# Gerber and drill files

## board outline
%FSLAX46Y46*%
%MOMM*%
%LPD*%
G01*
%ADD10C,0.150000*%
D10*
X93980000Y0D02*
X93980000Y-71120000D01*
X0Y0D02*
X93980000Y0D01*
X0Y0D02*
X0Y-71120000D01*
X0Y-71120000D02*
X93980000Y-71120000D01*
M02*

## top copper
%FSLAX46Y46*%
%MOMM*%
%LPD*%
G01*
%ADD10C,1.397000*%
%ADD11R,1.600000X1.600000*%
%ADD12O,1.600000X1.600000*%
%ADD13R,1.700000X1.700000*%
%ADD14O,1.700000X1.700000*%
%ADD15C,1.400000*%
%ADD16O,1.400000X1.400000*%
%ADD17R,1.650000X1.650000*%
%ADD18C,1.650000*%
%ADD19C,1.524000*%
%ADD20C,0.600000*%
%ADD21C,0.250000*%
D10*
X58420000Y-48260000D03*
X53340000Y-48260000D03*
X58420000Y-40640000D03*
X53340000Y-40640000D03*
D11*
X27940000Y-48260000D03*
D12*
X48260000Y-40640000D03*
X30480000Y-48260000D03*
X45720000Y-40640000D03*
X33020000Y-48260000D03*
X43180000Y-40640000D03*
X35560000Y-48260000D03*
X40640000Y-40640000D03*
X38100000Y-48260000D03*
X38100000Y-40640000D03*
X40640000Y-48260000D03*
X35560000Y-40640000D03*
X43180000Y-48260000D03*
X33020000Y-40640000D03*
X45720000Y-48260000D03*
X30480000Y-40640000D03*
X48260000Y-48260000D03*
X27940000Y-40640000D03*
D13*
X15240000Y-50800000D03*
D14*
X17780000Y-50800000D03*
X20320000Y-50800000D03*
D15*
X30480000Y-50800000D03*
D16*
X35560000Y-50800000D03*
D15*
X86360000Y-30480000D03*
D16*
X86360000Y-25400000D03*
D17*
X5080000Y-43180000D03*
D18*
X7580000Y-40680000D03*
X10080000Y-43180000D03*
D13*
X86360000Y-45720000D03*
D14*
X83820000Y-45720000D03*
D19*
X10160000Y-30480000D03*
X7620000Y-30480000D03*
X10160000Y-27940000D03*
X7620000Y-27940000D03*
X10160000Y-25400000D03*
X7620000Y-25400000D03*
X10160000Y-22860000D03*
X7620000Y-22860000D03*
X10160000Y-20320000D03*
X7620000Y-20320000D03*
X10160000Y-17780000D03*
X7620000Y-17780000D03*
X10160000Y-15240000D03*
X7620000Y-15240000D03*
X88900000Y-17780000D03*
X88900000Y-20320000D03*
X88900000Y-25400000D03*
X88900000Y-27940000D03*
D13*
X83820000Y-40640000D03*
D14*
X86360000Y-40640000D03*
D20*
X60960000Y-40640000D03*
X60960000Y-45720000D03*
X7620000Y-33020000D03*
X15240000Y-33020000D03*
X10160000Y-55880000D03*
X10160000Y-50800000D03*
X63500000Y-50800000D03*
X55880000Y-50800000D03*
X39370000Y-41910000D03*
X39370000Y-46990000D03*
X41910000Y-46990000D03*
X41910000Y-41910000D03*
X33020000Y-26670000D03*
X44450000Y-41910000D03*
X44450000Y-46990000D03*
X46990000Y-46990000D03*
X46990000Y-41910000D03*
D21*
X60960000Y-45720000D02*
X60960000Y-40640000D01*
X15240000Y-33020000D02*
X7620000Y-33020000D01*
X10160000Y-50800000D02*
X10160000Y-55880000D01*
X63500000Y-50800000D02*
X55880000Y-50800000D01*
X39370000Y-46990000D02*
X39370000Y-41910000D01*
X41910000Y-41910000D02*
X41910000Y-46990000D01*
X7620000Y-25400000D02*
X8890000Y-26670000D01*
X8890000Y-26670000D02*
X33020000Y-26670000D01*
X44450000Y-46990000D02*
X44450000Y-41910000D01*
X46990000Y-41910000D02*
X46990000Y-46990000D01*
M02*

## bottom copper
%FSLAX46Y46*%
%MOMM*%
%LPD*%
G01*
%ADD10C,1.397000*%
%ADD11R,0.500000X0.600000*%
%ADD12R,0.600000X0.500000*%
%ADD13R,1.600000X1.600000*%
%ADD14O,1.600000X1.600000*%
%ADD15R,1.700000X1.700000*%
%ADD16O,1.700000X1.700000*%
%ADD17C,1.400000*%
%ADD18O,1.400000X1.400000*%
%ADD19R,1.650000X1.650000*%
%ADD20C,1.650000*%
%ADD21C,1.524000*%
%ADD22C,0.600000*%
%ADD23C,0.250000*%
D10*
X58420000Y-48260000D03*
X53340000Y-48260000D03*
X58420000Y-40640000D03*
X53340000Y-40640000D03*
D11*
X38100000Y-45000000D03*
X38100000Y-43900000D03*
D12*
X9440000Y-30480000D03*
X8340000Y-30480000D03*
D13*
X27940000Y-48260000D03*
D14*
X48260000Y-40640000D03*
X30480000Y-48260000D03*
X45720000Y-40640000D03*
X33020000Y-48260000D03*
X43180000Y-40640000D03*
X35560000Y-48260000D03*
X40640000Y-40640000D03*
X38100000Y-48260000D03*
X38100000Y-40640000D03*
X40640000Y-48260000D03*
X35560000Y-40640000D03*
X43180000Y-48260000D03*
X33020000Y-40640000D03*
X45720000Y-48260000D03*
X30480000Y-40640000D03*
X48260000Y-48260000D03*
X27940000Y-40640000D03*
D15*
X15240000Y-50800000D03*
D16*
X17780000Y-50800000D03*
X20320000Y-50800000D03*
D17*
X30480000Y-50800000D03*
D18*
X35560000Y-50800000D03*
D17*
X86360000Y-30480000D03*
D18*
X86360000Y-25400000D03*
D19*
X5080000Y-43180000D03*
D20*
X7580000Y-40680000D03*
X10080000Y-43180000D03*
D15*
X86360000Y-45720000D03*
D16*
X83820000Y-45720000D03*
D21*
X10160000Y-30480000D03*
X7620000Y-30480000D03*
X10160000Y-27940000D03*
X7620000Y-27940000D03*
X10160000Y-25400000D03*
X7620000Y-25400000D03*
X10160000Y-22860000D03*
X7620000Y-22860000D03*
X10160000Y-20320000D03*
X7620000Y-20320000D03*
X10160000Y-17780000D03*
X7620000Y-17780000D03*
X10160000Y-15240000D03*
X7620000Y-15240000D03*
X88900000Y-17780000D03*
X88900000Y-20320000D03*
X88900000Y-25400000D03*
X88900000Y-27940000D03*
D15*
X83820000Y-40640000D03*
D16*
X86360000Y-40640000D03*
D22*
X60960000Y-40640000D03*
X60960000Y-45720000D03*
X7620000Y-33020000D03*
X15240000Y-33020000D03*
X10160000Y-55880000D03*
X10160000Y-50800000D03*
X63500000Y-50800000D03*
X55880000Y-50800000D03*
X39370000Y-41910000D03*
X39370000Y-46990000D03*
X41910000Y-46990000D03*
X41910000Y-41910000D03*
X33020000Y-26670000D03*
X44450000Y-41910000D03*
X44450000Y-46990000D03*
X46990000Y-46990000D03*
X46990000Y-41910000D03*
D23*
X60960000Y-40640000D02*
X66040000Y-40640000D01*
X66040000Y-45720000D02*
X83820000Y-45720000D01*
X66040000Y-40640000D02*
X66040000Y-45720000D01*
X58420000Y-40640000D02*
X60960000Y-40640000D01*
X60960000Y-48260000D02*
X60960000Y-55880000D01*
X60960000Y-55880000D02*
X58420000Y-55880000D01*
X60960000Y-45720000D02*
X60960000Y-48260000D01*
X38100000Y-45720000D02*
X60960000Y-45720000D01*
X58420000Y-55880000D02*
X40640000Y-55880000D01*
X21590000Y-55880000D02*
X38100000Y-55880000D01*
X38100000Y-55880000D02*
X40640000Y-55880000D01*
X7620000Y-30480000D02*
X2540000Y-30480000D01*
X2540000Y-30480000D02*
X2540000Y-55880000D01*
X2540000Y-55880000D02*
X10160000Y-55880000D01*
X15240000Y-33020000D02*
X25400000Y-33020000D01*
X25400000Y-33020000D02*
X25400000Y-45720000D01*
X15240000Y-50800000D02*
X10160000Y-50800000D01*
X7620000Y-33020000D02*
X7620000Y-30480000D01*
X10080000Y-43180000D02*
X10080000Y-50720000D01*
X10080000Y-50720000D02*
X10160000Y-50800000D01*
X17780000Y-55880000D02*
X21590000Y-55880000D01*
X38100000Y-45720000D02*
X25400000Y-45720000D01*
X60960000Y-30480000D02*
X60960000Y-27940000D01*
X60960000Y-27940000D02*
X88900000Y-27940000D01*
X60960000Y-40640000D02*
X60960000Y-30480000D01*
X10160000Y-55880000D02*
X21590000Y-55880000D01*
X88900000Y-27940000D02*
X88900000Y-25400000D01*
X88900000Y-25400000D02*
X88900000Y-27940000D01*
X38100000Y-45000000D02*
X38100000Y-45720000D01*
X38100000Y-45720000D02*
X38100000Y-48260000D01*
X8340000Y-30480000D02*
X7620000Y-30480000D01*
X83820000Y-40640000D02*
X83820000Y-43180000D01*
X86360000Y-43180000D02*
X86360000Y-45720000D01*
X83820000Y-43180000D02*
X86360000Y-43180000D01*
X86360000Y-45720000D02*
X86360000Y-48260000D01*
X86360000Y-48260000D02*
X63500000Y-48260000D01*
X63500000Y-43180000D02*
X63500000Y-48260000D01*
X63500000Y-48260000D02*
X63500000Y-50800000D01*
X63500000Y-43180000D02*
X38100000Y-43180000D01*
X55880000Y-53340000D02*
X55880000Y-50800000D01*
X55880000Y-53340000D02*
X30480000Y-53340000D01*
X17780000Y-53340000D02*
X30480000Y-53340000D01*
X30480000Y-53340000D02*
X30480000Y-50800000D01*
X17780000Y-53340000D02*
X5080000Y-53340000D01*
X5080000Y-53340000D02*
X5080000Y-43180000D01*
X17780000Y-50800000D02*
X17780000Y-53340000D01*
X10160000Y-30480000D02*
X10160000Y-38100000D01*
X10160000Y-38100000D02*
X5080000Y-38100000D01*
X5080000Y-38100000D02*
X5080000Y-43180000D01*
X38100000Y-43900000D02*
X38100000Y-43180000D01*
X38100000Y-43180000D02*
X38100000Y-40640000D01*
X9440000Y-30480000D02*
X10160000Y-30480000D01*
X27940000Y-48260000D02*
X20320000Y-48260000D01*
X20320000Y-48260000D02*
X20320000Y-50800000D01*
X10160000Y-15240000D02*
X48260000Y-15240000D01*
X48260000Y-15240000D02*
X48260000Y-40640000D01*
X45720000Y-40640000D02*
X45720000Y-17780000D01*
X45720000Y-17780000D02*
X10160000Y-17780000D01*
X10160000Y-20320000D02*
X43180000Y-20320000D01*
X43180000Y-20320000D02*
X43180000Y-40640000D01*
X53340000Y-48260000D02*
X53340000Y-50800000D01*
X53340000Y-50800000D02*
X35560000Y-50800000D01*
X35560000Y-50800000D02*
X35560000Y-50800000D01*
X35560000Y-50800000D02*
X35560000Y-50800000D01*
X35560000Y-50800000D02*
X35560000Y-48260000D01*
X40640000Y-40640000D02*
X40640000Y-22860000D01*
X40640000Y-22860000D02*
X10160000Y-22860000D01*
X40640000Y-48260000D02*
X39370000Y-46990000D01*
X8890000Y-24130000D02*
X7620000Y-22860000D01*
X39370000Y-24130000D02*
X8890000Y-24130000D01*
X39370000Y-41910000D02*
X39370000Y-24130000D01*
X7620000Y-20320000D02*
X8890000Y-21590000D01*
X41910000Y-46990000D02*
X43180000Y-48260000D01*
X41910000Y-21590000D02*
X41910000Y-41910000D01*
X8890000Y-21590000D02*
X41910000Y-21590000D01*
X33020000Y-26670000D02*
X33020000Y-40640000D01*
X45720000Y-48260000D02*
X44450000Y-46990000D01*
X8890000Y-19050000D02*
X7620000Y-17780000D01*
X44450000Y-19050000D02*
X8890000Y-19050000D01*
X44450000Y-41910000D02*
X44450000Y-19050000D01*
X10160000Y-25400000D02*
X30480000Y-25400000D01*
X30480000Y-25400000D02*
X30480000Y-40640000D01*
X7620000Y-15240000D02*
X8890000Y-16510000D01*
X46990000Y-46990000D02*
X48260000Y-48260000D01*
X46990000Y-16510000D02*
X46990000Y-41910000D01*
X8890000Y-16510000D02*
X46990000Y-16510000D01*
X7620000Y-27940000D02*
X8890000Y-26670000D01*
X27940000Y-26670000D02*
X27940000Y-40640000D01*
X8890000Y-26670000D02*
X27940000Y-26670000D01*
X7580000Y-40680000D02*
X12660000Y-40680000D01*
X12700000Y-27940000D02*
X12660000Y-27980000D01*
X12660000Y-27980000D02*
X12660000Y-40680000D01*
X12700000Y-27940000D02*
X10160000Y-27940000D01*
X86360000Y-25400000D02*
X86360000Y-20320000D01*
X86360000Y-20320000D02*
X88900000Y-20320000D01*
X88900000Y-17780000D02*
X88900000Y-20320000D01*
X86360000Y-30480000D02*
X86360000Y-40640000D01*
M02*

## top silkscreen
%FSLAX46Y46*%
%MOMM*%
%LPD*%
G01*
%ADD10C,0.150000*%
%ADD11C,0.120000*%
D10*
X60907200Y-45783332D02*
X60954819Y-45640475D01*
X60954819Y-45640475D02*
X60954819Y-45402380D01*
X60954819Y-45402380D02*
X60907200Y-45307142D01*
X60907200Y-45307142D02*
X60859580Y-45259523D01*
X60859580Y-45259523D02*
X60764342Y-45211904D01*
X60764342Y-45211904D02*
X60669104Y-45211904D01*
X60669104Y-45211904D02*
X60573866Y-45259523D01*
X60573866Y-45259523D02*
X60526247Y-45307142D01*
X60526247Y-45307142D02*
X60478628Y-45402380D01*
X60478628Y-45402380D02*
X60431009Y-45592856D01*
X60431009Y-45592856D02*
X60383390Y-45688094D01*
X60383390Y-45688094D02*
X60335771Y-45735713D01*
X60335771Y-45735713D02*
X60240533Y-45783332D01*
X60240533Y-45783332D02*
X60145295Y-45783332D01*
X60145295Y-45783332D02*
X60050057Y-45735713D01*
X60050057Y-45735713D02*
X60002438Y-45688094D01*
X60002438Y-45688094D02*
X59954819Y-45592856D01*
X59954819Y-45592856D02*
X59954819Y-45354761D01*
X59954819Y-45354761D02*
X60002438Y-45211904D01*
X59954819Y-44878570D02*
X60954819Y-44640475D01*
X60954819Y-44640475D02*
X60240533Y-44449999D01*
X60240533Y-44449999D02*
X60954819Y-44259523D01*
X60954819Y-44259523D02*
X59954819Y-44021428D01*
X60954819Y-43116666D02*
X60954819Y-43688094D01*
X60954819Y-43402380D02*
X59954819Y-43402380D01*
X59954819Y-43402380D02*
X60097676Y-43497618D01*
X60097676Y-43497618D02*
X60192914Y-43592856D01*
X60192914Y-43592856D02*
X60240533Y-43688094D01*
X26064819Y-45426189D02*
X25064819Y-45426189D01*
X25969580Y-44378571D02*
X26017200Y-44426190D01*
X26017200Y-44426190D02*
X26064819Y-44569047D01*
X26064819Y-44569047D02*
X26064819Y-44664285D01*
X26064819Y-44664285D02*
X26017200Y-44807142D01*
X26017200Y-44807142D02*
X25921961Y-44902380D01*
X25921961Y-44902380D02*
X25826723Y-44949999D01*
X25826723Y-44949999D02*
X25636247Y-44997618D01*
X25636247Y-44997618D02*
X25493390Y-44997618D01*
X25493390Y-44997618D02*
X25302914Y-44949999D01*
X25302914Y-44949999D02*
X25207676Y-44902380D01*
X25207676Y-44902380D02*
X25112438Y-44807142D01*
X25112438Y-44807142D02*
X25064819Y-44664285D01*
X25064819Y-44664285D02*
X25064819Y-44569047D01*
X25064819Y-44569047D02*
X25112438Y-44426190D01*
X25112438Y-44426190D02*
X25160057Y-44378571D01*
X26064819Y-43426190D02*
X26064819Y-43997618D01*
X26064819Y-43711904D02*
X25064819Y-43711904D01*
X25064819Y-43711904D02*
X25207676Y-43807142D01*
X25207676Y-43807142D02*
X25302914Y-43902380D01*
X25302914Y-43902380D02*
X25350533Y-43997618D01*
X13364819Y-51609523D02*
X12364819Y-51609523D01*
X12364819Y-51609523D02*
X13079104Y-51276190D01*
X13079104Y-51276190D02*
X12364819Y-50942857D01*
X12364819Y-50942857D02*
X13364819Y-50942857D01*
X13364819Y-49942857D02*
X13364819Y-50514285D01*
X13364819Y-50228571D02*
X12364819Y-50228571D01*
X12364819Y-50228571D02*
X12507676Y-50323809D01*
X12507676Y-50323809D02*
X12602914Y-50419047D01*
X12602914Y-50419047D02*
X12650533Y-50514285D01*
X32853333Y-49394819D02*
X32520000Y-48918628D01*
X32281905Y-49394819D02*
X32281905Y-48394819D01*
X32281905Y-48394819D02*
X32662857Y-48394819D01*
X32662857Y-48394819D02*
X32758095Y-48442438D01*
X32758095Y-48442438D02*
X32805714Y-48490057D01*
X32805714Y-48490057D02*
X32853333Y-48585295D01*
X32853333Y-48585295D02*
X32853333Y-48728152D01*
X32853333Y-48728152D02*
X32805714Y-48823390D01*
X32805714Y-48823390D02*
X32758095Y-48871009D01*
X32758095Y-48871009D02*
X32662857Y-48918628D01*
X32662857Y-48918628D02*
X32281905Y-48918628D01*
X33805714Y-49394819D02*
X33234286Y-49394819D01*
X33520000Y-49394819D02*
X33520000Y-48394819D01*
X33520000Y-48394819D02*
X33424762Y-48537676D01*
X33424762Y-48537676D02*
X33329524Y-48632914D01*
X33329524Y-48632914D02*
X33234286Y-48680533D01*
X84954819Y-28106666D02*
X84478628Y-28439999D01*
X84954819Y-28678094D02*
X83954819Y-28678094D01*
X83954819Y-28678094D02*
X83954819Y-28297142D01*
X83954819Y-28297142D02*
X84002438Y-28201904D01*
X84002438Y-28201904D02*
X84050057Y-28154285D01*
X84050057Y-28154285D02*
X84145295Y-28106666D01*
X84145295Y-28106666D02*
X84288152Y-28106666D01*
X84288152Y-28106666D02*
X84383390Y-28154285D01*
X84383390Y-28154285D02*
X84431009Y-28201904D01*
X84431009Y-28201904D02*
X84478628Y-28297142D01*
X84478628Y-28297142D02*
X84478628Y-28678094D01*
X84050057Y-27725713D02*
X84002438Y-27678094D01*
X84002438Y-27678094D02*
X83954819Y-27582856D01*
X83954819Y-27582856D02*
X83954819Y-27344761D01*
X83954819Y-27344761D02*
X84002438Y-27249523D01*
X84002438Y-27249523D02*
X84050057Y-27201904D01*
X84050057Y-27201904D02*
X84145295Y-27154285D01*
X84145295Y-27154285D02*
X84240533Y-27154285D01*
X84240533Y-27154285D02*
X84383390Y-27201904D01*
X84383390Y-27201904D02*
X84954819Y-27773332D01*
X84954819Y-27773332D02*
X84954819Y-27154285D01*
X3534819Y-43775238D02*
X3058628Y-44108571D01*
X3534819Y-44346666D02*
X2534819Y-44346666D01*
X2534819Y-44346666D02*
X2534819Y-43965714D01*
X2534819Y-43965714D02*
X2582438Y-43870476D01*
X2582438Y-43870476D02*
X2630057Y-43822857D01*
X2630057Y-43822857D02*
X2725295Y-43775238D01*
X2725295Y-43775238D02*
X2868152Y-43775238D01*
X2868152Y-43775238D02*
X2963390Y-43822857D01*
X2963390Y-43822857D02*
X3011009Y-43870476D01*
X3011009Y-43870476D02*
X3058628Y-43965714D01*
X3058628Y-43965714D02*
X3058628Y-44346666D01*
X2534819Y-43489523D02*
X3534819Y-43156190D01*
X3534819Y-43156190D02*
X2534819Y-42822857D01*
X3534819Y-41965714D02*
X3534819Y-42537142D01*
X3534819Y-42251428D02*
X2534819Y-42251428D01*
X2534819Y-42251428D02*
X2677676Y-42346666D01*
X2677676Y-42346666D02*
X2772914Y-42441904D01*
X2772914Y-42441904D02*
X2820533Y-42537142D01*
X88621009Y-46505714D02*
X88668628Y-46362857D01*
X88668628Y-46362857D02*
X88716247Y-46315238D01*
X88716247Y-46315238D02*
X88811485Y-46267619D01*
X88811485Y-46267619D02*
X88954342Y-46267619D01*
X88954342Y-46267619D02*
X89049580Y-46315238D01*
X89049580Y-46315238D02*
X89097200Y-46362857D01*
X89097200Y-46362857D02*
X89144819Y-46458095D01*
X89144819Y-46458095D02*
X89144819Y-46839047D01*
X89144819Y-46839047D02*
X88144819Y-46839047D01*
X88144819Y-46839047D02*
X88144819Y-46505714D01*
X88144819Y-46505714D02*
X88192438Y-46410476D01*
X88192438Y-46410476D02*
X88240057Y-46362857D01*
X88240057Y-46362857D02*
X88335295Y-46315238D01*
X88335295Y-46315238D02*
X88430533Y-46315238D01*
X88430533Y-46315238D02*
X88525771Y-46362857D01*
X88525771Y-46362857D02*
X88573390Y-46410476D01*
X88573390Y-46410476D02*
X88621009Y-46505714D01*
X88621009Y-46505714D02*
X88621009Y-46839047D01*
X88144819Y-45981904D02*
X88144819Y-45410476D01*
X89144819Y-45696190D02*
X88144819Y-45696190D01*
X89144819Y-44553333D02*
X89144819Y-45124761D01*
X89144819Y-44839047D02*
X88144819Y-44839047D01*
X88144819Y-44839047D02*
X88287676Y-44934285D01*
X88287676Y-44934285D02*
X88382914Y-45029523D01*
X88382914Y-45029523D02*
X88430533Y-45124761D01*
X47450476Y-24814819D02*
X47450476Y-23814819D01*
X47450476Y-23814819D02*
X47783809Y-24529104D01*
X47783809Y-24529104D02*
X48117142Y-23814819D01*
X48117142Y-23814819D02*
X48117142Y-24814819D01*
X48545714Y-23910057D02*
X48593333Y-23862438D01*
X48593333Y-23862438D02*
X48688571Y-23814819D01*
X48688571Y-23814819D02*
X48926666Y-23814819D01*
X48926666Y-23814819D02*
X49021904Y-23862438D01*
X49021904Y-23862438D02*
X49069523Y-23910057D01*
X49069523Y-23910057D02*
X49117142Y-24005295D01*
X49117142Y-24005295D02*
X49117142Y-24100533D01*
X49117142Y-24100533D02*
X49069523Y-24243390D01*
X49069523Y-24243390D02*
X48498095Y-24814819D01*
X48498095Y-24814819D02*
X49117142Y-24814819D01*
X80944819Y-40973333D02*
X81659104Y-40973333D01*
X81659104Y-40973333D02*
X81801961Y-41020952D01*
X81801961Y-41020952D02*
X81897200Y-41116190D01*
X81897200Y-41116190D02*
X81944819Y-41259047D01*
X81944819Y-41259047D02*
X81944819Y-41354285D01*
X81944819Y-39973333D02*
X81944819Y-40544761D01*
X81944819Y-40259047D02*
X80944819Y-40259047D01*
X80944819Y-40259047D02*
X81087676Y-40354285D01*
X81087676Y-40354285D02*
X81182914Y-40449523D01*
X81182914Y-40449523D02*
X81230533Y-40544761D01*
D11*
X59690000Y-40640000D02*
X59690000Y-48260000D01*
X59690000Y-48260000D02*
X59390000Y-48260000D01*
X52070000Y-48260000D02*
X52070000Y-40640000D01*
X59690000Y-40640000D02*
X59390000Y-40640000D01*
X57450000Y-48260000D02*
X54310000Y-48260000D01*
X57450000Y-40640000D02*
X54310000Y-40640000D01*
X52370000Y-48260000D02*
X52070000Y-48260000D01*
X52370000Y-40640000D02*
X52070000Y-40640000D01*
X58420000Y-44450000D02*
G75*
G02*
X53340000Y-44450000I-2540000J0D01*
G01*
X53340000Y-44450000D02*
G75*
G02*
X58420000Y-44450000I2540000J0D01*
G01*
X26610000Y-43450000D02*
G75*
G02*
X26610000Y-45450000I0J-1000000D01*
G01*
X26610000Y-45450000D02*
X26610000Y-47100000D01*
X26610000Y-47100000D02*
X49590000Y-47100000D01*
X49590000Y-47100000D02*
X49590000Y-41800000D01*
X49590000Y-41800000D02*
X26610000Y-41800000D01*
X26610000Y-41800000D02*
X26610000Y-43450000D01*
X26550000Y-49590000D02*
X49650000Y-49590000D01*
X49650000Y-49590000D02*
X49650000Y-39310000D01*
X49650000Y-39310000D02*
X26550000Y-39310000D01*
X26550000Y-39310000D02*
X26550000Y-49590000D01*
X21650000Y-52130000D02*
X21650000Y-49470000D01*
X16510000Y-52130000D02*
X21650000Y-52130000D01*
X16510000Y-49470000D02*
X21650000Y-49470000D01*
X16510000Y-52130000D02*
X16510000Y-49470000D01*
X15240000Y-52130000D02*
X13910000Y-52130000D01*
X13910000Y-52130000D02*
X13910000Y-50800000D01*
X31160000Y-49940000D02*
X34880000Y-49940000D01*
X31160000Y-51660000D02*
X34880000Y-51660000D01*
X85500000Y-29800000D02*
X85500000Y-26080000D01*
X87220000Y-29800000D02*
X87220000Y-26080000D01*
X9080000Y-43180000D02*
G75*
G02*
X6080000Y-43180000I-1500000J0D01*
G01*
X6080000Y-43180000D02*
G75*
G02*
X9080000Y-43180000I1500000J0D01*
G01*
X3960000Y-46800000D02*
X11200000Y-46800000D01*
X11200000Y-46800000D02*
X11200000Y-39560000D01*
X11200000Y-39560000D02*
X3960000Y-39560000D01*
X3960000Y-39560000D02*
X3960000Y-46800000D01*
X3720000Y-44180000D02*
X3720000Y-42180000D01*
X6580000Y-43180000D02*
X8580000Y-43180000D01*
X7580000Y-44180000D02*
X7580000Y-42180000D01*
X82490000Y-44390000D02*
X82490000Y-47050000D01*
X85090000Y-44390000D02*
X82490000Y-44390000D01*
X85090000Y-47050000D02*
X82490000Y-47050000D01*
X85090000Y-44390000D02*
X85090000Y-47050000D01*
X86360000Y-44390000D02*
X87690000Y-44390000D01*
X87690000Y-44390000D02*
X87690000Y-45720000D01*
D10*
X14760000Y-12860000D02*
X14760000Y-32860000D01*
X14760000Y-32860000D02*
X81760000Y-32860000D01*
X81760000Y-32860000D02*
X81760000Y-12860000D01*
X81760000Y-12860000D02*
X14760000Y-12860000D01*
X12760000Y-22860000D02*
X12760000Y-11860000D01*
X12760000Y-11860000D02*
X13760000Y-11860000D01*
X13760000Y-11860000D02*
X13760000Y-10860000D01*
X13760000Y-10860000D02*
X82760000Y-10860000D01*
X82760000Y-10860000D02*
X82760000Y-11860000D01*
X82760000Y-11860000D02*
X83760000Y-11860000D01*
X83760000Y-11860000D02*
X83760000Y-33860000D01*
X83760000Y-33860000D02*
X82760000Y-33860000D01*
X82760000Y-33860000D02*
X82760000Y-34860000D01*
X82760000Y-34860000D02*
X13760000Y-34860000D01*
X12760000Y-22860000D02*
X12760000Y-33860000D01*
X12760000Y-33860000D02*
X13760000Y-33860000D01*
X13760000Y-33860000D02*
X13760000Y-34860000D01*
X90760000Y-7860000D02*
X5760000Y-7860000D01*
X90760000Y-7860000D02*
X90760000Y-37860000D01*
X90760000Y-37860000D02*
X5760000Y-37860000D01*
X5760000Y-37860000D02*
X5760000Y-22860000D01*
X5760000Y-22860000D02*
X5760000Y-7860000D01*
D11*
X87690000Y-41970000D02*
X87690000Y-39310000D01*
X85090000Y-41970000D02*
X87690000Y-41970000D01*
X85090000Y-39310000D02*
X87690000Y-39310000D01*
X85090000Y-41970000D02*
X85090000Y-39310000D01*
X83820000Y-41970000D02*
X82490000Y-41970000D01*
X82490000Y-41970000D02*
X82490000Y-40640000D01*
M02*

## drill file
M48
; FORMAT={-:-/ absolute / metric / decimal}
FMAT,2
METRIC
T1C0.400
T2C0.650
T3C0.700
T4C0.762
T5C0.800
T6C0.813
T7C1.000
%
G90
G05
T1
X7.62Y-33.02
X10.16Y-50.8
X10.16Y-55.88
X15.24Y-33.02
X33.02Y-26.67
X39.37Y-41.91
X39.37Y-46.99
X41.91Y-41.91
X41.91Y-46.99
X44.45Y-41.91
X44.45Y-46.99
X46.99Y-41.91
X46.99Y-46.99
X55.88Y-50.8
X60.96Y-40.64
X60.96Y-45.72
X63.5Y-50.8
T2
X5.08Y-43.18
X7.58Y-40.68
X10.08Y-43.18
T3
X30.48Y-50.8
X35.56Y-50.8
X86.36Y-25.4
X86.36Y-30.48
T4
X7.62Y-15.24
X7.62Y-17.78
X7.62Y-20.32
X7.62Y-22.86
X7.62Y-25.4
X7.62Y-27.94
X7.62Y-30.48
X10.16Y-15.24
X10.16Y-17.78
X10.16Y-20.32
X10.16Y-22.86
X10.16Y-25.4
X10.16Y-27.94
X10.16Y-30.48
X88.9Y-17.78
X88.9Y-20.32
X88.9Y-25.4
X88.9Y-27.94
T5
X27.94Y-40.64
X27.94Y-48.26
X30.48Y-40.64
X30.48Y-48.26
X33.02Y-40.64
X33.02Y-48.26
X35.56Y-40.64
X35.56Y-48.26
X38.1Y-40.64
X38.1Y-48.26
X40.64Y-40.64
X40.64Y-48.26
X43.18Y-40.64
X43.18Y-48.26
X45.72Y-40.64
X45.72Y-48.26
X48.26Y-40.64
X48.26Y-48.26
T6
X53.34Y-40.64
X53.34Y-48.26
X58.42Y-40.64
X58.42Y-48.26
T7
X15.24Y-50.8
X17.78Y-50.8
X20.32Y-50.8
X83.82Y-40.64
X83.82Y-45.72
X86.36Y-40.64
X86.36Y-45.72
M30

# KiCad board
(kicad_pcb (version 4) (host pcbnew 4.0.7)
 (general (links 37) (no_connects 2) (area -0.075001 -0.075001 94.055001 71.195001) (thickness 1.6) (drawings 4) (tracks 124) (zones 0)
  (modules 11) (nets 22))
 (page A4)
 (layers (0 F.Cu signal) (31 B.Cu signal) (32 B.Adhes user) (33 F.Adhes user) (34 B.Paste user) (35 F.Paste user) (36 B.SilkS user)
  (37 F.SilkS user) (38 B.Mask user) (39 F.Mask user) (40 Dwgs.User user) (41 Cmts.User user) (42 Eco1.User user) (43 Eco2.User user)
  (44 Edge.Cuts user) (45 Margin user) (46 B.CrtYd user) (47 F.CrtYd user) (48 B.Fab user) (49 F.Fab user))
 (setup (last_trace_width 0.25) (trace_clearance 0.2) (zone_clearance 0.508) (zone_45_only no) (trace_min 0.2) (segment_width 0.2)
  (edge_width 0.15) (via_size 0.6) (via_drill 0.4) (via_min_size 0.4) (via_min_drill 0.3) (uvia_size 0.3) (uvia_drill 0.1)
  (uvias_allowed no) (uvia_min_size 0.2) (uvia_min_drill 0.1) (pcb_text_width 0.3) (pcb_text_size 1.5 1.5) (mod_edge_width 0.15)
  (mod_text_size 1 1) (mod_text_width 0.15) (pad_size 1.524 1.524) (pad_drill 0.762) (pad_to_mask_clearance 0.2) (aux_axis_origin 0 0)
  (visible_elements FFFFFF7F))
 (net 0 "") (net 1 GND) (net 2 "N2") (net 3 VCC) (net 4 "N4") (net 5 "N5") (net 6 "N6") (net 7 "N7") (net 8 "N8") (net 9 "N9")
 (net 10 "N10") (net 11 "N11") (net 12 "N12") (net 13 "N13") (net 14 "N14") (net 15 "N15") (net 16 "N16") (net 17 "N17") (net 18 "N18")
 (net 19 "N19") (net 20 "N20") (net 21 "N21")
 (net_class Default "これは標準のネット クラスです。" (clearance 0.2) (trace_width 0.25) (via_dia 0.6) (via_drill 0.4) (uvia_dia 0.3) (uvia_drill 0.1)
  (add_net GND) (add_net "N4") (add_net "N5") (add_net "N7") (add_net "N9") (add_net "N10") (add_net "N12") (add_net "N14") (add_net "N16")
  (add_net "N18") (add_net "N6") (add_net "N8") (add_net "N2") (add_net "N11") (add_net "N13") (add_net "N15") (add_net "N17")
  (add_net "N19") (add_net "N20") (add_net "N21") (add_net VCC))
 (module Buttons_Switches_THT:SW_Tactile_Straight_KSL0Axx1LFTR (layer F.Cu) (at 58.42 40.64 270)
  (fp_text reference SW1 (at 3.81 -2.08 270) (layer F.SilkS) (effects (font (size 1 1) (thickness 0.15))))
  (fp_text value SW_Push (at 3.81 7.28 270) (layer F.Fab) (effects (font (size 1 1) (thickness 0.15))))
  (fp_line (start 0 -1.27) (end 7.62 -1.27) (layer F.SilkS) (width 0.12))
  (fp_line (start 7.62 -1.27) (end 7.62 -0.97) (layer F.SilkS) (width 0.12))
  (fp_line (start 7.62 6.35) (end 0 6.35) (layer F.SilkS) (width 0.12))
  (fp_line (start 0 -1.27) (end 0 -0.97) (layer F.SilkS) (width 0.12))
  (fp_line (start 7.62 0.97) (end 7.62 4.11) (layer F.SilkS) (width 0.12))
  (fp_line (start 0 0.97) (end 0 4.11) (layer F.SilkS) (width 0.12))
  (fp_line (start 7.62 6.05) (end 7.62 6.35) (layer F.SilkS) (width 0.12))
  (fp_line (start 0 6.05) (end 0 6.35) (layer F.SilkS) (width 0.12))
  (fp_circle (center 3.81 2.54) (end 3.81 0) (layer F.SilkS) (width 0.12))
  (pad 1 thru_hole circle (at 7.62 0 270) (size 1.397 1.397) (drill 0.8128) (layers *.Cu *.Mask) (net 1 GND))
  (pad 2 thru_hole circle (at 7.62 5.08 270) (size 1.397 1.397) (drill 0.8128) (layers *.Cu *.Mask) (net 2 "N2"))
  (pad 1 thru_hole circle (at 0 0 270) (size 1.397 1.397) (drill 0.8128) (layers *.Cu *.Mask) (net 1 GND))
  (pad 2 thru_hole circle (at 0 5.08 270) (size 1.397 1.397) (drill 0.8128) (layers *.Cu *.Mask) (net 2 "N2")))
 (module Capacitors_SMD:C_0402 (layer B.Cu) (at 38.1 44.45 90)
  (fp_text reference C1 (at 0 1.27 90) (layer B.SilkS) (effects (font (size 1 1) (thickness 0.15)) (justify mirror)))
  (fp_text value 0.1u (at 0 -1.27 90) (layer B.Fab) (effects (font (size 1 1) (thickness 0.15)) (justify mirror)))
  (pad 1 smd rect (at -0.55 0 90) (size 0.6 0.5) (layers B.Cu B.Paste B.Mask) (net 1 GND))
  (pad 2 smd rect (at 0.55 0 90) (size 0.6 0.5) (layers B.Cu B.Paste B.Mask) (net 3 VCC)))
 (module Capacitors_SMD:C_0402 (layer B.Cu) (at 8.89 30.48 180)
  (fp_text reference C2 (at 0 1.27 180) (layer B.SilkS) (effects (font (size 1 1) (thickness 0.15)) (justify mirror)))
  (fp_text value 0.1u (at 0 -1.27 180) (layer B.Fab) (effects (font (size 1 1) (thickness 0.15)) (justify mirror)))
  (pad 1 smd rect (at -0.55 0 180) (size 0.6 0.5) (layers B.Cu B.Paste B.Mask) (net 3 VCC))
  (pad 2 smd rect (at 0.55 0 180) (size 0.6 0.5) (layers B.Cu B.Paste B.Mask) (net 1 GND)))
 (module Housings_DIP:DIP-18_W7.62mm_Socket (layer F.Cu) (at 27.94 48.26 90)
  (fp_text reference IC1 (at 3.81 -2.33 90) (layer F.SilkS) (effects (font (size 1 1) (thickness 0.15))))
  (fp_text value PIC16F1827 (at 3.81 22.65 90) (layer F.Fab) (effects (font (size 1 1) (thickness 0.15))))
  (fp_arc (start 3.81 -1.33) (end 2.81 -1.33) (angle -180) (layer F.SilkS) (width 0.12))
  (fp_line (start 2.81 -1.33) (end 1.16 -1.33) (layer F.SilkS) (width 0.12))
  (fp_line (start 1.16 -1.33) (end 1.16 21.65) (layer F.SilkS) (width 0.12))
  (fp_line (start 1.16 21.65) (end 6.46 21.65) (layer F.SilkS) (width 0.12))
  (fp_line (start 6.46 21.65) (end 6.46 -1.33) (layer F.SilkS) (width 0.12))
  (fp_line (start 6.46 -1.33) (end 4.81 -1.33) (layer F.SilkS) (width 0.12))
  (fp_line (start -1.33 -1.39) (end -1.33 21.71) (layer F.SilkS) (width 0.12))
  (fp_line (start -1.33 21.71) (end 8.95 21.71) (layer F.SilkS) (width 0.12))
  (fp_line (start 8.95 21.71) (end 8.95 -1.39) (layer F.SilkS) (width 0.12))
  (fp_line (start 8.95 -1.39) (end -1.33 -1.39) (layer F.SilkS) (width 0.12))
  (pad 1 thru_hole rect (at 0 0 90) (size 1.6 1.6) (drill 0.8) (layers *.Cu *.Mask) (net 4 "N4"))
  (pad 10 thru_hole oval (at 7.62 20.32 90) (size 1.6 1.6) (drill 0.8) (layers *.Cu *.Mask) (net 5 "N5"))
  (pad 2 thru_hole oval (at 0 2.54 90) (size 1.6 1.6) (drill 0.8) (layers *.Cu *.Mask) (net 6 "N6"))
  (pad 11 thru_hole oval (at 7.62 17.78 90) (size 1.6 1.6) (drill 0.8) (layers *.Cu *.Mask) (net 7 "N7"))
  (pad 3 thru_hole oval (at 0 5.08 90) (size 1.6 1.6) (drill 0.8) (layers *.Cu *.Mask) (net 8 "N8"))
  (pad 12 thru_hole oval (at 7.62 15.24 90) (size 1.6 1.6) (drill 0.8) (layers *.Cu *.Mask) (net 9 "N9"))
  (pad 4 thru_hole oval (at 0 7.62 90) (size 1.6 1.6) (drill 0.8) (layers *.Cu *.Mask) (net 2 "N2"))
  (pad 13 thru_hole oval (at 7.62 12.7 90) (size 1.6 1.6) (drill 0.8) (layers *.Cu *.Mask) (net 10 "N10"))
  (pad 5 thru_hole oval (at 0 10.16 90) (size 1.6 1.6) (drill 0.8) (layers *.Cu *.Mask) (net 1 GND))
  (pad 14 thru_hole oval (at 7.62 10.16 90) (size 1.6 1.6) (drill 0.8) (layers *.Cu *.Mask) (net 3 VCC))
  (pad 6 thru_hole oval (at 0 12.7 90) (size 1.6 1.6) (drill 0.8) (layers *.Cu *.Mask) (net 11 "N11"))
  (pad 15 thru_hole oval (at 7.62 7.62 90) (size 1.6 1.6) (drill 0.8) (layers *.Cu *.Mask) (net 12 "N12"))
  (pad 7 thru_hole oval (at 0 15.24 90) (size 1.6 1.6) (drill 0.8) (layers *.Cu *.Mask) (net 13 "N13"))
  (pad 16 thru_hole oval (at 7.62 5.08 90) (size 1.6 1.6) (drill 0.8) (layers *.Cu *.Mask) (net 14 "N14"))
  (pad 8 thru_hole oval (at 0 17.78 90) (size 1.6 1.6) (drill 0.8) (layers *.Cu *.Mask) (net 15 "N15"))
  (pad 17 thru_hole oval (at 7.62 2.54 90) (size 1.6 1.6) (drill 0.8) (layers *.Cu *.Mask) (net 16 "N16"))
  (pad 9 thru_hole oval (at 0 20.32 90) (size 1.6 1.6) (drill 0.8) (layers *.Cu *.Mask) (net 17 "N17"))
  (pad 18 thru_hole oval (at 7.62 0 90) (size 1.6 1.6) (drill 0.8) (layers *.Cu *.Mask) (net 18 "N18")))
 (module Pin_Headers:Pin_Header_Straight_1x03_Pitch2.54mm (layer F.Cu) (at 15.24 50.8 90)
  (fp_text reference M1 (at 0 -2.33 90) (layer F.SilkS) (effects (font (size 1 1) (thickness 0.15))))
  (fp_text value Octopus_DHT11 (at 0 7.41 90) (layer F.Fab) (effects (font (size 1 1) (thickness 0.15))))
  (fp_line (start -1.33 6.41) (end 1.33 6.41) (layer F.SilkS) (width 0.12))
  (fp_line (start -1.33 1.27) (end -1.33 6.41) (layer F.SilkS) (width 0.12))
  (fp_line (start 1.33 1.27) (end 1.33 6.41) (layer F.SilkS) (width 0.12))
  (fp_line (start -1.33 1.27) (end 1.33 1.27) (layer F.SilkS) (width 0.12))
  (fp_line (start -1.33 0) (end -1.33 -1.33) (layer F.SilkS) (width 0.12))
  (fp_line (start -1.33 -1.33) (end 0 -1.33) (layer F.SilkS) (width 0.12))
  (pad 1 thru_hole rect (at 0 0 90) (size 1.7 1.7) (drill 1) (layers *.Cu *.Mask) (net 1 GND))
  (pad 2 thru_hole oval (at 0 2.54 90) (size 1.7 1.7) (drill 1) (layers *.Cu *.Mask) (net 3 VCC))
  (pad 3 thru_hole oval (at 0 5.08 90) (size 1.7 1.7) (drill 1) (layers *.Cu *.Mask) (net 4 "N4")))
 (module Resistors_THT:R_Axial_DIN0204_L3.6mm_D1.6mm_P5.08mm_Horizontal (layer F.Cu) (at 30.48 50.8)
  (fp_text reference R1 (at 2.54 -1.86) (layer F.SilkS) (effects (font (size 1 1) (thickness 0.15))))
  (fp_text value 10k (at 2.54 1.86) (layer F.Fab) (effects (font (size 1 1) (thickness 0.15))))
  (fp_line (start 0.68 -0.86) (end 4.4 -0.86) (layer F.SilkS) (width 0.12))
  (fp_line (start 0.68 0.86) (end 4.4 0.86) (layer F.SilkS) (width 0.12))
  (pad 1 thru_hole circle (at 0 0) (size 1.4 1.4) (drill 0.7) (layers *.Cu *.Mask) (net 3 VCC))
  (pad 2 thru_hole oval (at 5.08 0) (size 1.4 1.4) (drill 0.7) (layers *.Cu *.Mask) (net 2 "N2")))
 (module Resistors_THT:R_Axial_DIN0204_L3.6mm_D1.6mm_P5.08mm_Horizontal (layer F.Cu) (at 86.36 30.48 90)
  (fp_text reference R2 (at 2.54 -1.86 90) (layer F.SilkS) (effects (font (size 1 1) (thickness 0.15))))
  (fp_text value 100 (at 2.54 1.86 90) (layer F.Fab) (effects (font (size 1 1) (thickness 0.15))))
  (fp_line (start 0.68 -0.86) (end 4.4 -0.86) (layer F.SilkS) (width 0.12))
  (fp_line (start 0.68 0.86) (end 4.4 0.86) (layer F.SilkS) (width 0.12))
  (pad 1 thru_hole circle (at 0 0 90) (size 1.4 1.4) (drill 0.7) (layers *.Cu *.Mask) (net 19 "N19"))
  (pad 2 thru_hole oval (at 5.08 0 90) (size 1.4 1.4) (drill 0.7) (layers *.Cu *.Mask) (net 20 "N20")))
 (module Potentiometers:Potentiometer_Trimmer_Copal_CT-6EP (layer F.Cu) (at 5.08 43.18 90)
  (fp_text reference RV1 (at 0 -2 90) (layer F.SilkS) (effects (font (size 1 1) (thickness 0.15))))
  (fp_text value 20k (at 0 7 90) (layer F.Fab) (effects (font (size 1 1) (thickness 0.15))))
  (fp_circle (center 0 2.5) (end 1.5 2.5) (layer F.SilkS) (width 0.12))
  (fp_line (start -3.62 -1.12) (end -3.62 6.12) (layer F.SilkS) (width 0.12))
  (fp_line (start -3.62 6.12) (end 3.62 6.12) (layer F.SilkS) (width 0.12))
  (fp_line (start 3.62 6.12) (end 3.62 -1.12) (layer F.SilkS) (width 0.12))
  (fp_line (start 3.62 -1.12) (end -3.62 -1.12) (layer F.SilkS) (width 0.12))
  (fp_line (start -1 -1.36) (end 1 -1.36) (layer F.SilkS) (width 0.12))
  (fp_line (start 0 1.5) (end 0 3.5) (layer F.SilkS) (width 0.12))
  (fp_line (start -1 2.5) (end 1 2.5) (layer F.SilkS) (width 0.12))
  (pad 1 thru_hole rect (at 0 0 90) (size 1.65 1.65) (drill 0.65) (layers *.Cu *.Mask) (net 3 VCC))
  (pad 2 thru_hole circle (at 2.5 2.5 90) (size 1.65 1.65) (drill 0.65) (layers *.Cu *.Mask) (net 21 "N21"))
  (pad 3 thru_hole circle (at 0 5 90) (size 1.65 1.65) (drill 0.65) (layers *.Cu *.Mask) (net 1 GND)))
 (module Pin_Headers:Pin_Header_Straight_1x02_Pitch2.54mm (layer F.Cu) (at 86.36 45.72 270)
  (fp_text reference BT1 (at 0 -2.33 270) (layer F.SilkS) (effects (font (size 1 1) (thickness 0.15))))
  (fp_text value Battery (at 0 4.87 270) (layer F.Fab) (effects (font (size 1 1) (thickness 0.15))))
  (fp_line (start -1.33 3.87) (end 1.33 3.87) (layer F.SilkS) (width 0.12))
  (fp_line (start -1.33 1.27) (end -1.33 3.87) (layer F.SilkS) (width 0.12))
  (fp_line (start 1.33 1.27) (end 1.33 3.87) (layer F.SilkS) (width 0.12))
  (fp_line (start -1.33 1.27) (end 1.33 1.27) (layer F.SilkS) (width 0.12))
  (fp_line (start -1.33 0) (end -1.33 -1.33) (layer F.SilkS) (width 0.12))
  (fp_line (start -1.33 -1.33) (end 0 -1.33) (layer F.SilkS) (width 0.12))
  (pad 1 thru_hole rect (at 0 0 270) (size 1.7 1.7) (drill 1) (layers *.Cu *.Mask) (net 3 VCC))
  (pad 2 thru_hole oval (at 0 2.54 270) (size 1.7 1.7) (drill 1) (layers *.Cu *.Mask) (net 1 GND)))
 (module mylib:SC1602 (layer F.Cu) (at 48.26 22.86)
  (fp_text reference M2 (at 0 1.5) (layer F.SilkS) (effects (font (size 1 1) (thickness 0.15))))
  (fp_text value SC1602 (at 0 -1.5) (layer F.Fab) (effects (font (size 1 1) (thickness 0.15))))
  (fp_line (start -33.5 -10) (end -33.5 10) (layer F.SilkS) (width 0.15))
  (fp_line (start -33.5 10) (end 33.5 10) (layer F.SilkS) (width 0.15))
  (fp_line (start 33.5 10) (end 33.5 -10) (layer F.SilkS) (width 0.15))
  (fp_line (start 33.5 -10) (end -33.5 -10) (layer F.SilkS) (width 0.15))
  (fp_line (start -35.5 0) (end -35.5 -11) (layer F.SilkS) (width 0.15))
  (fp_line (start -35.5 -11) (end -34.5 -11) (layer F.SilkS) (width 0.15))
  (fp_line (start -34.5 -11) (end -34.5 -12) (layer F.SilkS) (width 0.15))
  (fp_line (start -34.5 -12) (end 34.5 -12) (layer F.SilkS) (width 0.15))
  (fp_line (start 34.5 -12) (end 34.5 -11) (layer F.SilkS) (width 0.15))
  (fp_line (start 34.5 -11) (end 35.5 -11) (layer F.SilkS) (width 0.15))
  (fp_line (start 35.5 -11) (end 35.5 11) (layer F.SilkS) (width 0.15))
  (fp_line (start 35.5 11) (end 34.5 11) (layer F.SilkS) (width 0.15))
  (fp_line (start 34.5 11) (end 34.5 12) (layer F.SilkS) (width 0.15))
  (fp_line (start 34.5 12) (end -34.5 12) (layer F.SilkS) (width 0.15))
  (fp_line (start -35.5 0) (end -35.5 11) (layer F.SilkS) (width 0.15))
  (fp_line (start -35.5 11) (end -34.5 11) (layer F.SilkS) (width 0.15))
  (fp_line (start -34.5 11) (end -34.5 12) (layer F.SilkS) (width 0.15))
  (fp_line (start 42.5 -15) (end -42.5 -15) (layer F.SilkS) (width 0.15))
  (fp_line (start 42.5 -15) (end 42.5 15) (layer F.SilkS) (width 0.15))
  (fp_line (start 42.5 15) (end -42.5 15) (layer F.SilkS) (width 0.15))
  (fp_line (start -42.5 15) (end -42.5 0) (layer F.SilkS) (width 0.15))
  (fp_line (start -42.5 0) (end -42.5 -15) (layer F.SilkS) (width 0.15))
  (pad 1 thru_hole circle (at -38.1 7.62) (size 1.524 1.524) (drill 0.762) (layers *.Cu *.Mask) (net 3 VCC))
  (pad 2 thru_hole circle (at -40.64 7.62) (size 1.524 1.524) (drill 0.762) (layers *.Cu *.Mask) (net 1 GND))
  (pad 3 thru_hole circle (at -38.1 5.08) (size 1.524 1.524) (drill 0.762) (layers *.Cu *.Mask) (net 21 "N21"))
  (pad 4 thru_hole circle (at -40.64 5.08) (size 1.524 1.524) (drill 0.762) (layers *.Cu *.Mask) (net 18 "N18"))
  (pad 5 thru_hole circle (at -38.1 2.54) (size 1.524 1.524) (drill 0.762) (layers *.Cu *.Mask) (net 16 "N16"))
  (pad 6 thru_hole circle (at -40.64 2.54) (size 1.524 1.524) (drill 0.762) (layers *.Cu *.Mask) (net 14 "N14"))
  (pad 7 thru_hole circle (at -38.1 0) (size 1.524 1.524) (drill 0.762) (layers *.Cu *.Mask) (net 10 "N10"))
  (pad 8 thru_hole circle (at -40.64 0) (size 1.524 1.524) (drill 0.762) (layers *.Cu *.Mask) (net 11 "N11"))
  (pad 9 thru_hole circle (at -38.1 -2.54) (size 1.524 1.524) (drill 0.762) (layers *.Cu *.Mask) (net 9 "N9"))
  (pad 10 thru_hole circle (at -40.64 -2.54) (size 1.524 1.524) (drill 0.762) (layers *.Cu *.Mask) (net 13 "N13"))
  (pad 11 thru_hole circle (at -38.1 -5.08) (size 1.524 1.524) (drill 0.762) (layers *.Cu *.Mask) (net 7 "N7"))
  (pad 12 thru_hole circle (at -40.64 -5.08) (size 1.524 1.524) (drill 0.762) (layers *.Cu *.Mask) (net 15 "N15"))
  (pad 13 thru_hole circle (at -38.1 -7.62) (size 1.524 1.524) (drill 0.762) (layers *.Cu *.Mask) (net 5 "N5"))
  (pad 14 thru_hole circle (at -40.64 -7.62) (size 1.524 1.524) (drill 0.762) (layers *.Cu *.Mask) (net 17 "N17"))
  (pad 15 thru_hole circle (at 40.64 -5.08) (size 1.524 1.524) (drill 0.762) (layers *.Cu *.Mask) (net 20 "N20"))
  (pad 15 thru_hole circle (at 40.64 -2.54) (size 1.524 1.524) (drill 0.762) (layers *.Cu *.Mask) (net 20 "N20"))
  (pad 16 thru_hole circle (at 40.64 2.54) (size 1.524 1.524) (drill 0.762) (layers *.Cu *.Mask) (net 1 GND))
  (pad 16 thru_hole circle (at 40.64 5.08) (size 1.524 1.524) (drill 0.762) (layers *.Cu *.Mask) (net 1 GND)))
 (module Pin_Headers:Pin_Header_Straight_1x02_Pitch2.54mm (layer F.Cu) (at 83.82 40.64 90)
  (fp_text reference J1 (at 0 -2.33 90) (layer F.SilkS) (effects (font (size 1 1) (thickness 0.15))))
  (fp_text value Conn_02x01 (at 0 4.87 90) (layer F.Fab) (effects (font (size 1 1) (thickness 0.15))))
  (fp_line (start -1.33 3.87) (end 1.33 3.87) (layer F.SilkS) (width 0.12))
  (fp_line (start -1.33 1.27) (end -1.33 3.87) (layer F.SilkS) (width 0.12))
  (fp_line (start 1.33 1.27) (end 1.33 3.87) (layer F.SilkS) (width 0.12))
  (fp_line (start -1.33 1.27) (end 1.33 1.27) (layer F.SilkS) (width 0.12))
  (fp_line (start -1.33 0) (end -1.33 -1.33) (layer F.SilkS) (width 0.12))
  (fp_line (start -1.33 -1.33) (end 0 -1.33) (layer F.SilkS) (width 0.12))
  (pad 1 thru_hole rect (at 0 0 90) (size 1.7 1.7) (drill 1) (layers *.Cu *.Mask) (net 3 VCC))
  (pad 2 thru_hole oval (at 0 2.54 90) (size 1.7 1.7) (drill 1) (layers *.Cu *.Mask) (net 19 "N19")))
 (gr_line (start 93.98 0) (end 93.98 71.12) (angle 90) (layer Edge.Cuts) (width 0.15))
 (gr_line (start 0 0) (end 93.98 0) (angle 90) (layer Edge.Cuts) (width 0.15))
 (gr_line (start 0 0) (end 0 71.12) (angle 90) (layer Edge.Cuts) (width 0.15))
 (gr_line (start 0 71.12) (end 93.98 71.12) (angle 90) (layer Edge.Cuts) (width 0.15))
 (segment (start 60.96 40.64) (end 66.04 40.64) (width 0.25) (layer B.Cu) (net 1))
 (segment (start 66.04 45.72) (end 83.82 45.72) (width 0.25) (layer B.Cu) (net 1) (status 800000))
 (segment (start 66.04 40.64) (end 66.04 45.72) (width 0.25) (layer B.Cu) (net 1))
 (segment (start 58.42 40.64) (end 60.96 40.64) (width 0.25) (layer B.Cu) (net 1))
 (segment (start 60.96 48.26) (end 60.96 55.88) (width 0.25) (layer B.Cu) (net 1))
 (segment (start 60.96 55.88) (end 58.42 55.88) (width 0.25) (layer B.Cu) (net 1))
 (segment (start 60.96 45.72) (end 60.96 48.26) (width 0.25) (layer B.Cu) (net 1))
 (via (at 60.96 40.64) (size 0.6) (drill 0.4) (layers F.Cu B.Cu) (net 1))
 (segment (start 38.1 45.72) (end 60.96 45.72) (width 0.25) (layer B.Cu) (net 1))
 (via (at 60.96 45.72) (size 0.6) (drill 0.4) (layers F.Cu B.Cu) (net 1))
 (segment (start 60.96 45.72) (end 60.96 40.64) (width 0.25) (layer F.Cu) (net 1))
 (segment (start 58.42 55.88) (end 40.64 55.88) (width 0.25) (layer B.Cu) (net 1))
 (segment (start 21.59 55.88) (end 38.1 55.88) (width 0.25) (layer B.Cu) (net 1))
 (segment (start 38.1 55.88) (end 40.64 55.88) (width 0.25) (layer B.Cu) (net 1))
 (segment (start 7.62 30.48) (end 2.54 30.48) (width 0.25) (layer B.Cu) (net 1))
 (segment (start 2.54 30.48) (end 2.54 55.88) (width 0.25) (layer B.Cu) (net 1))
 (segment (start 2.54 55.88) (end 10.16 55.88) (width 0.25) (layer B.Cu) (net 1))
 (segment (start 15.24 33.02) (end 25.4 33.02) (width 0.25) (layer B.Cu) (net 1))
 (segment (start 25.4 33.02) (end 25.4 45.72) (width 0.25) (layer B.Cu) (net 1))
 (segment (start 15.24 50.8) (end 10.16 50.8) (width 0.25) (layer B.Cu) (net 1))
 (segment (start 7.62 33.02) (end 7.62 30.48) (width 0.25) (layer B.Cu) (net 1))
 (via (at 7.62 33.02) (size 0.6) (drill 0.4) (layers F.Cu B.Cu) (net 1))
 (segment (start 15.24 33.02) (end 7.62 33.02) (width 0.25) (layer F.Cu) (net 1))
 (via (at 15.24 33.02) (size 0.6) (drill 0.4) (layers F.Cu B.Cu) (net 1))
 (segment (start 10.08 43.18) (end 10.08 50.72) (width 0.25) (layer B.Cu) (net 1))
 (via (at 10.16 55.88) (size 0.6) (drill 0.4) (layers F.Cu B.Cu) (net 1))
 (segment (start 10.16 50.8) (end 10.16 55.88) (width 0.25) (layer F.Cu) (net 1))
 (via (at 10.16 50.8) (size 0.6) (drill 0.4) (layers F.Cu B.Cu) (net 1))
 (segment (start 10.08 50.72) (end 10.16 50.8) (width 0.25) (layer B.Cu) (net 1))
 (segment (start 17.78 55.88) (end 21.59 55.88) (width 0.25) (layer B.Cu) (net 1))
 (segment (start 38.1 45.72) (end 25.4 45.72) (width 0.25) (layer B.Cu) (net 1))
 (segment (start 60.96 30.48) (end 60.96 27.94) (width 0.25) (layer B.Cu) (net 1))
 (segment (start 60.96 27.94) (end 88.9 27.94) (width 0.25) (layer B.Cu) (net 1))
 (segment (start 60.96 40.64) (end 60.96 30.48) (width 0.25) (layer B.Cu) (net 1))
 (segment (start 10.16 55.88) (end 21.59 55.88) (width 0.25) (layer B.Cu) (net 1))
 (segment (start 88.9 27.94) (end 88.9 25.4) (width 0.25) (layer B.Cu) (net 1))
 (segment (start 88.9 25.4) (end 88.9 27.94) (width 0.25) (layer B.Cu) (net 1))
 (segment (start 38.1 45) (end 38.1 45.72) (width 0.25) (layer B.Cu) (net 1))
 (segment (start 38.1 45.72) (end 38.1 48.26) (width 0.25) (layer B.Cu) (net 1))
 (segment (start 8.34 30.48) (end 7.62 30.48) (width 0.25) (layer B.Cu) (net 1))
 (segment (start 83.82 40.64) (end 83.82 43.18) (width 0.25) (layer B.Cu) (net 3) (status 400000))
 (segment (start 86.36 43.18) (end 86.36 45.72) (width 0.25) (layer B.Cu) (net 3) (status 800000))
 (segment (start 83.82 43.18) (end 86.36 43.18) (width 0.25) (layer B.Cu) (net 3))
 (segment (start 86.36 45.72) (end 86.36 48.26) (width 0.25) (layer B.Cu) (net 3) (status 400000))
 (segment (start 86.36 48.26) (end 63.5 48.26) (width 0.25) (layer B.Cu) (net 3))
 (segment (start 63.5 43.18) (end 63.5 48.26) (width 0.25) (layer B.Cu) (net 3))
 (segment (start 63.5 48.26) (end 63.5 50.8) (width 0.25) (layer B.Cu) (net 3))
 (via (at 63.5 50.8) (size 0.6) (drill 0.4) (layers F.Cu B.Cu) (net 3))
 (segment (start 63.5 43.18) (end 38.1 43.18) (width 0.25) (layer B.Cu) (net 3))
 (via (at 55.88 50.8) (size 0.6) (drill 0.4) (layers F.Cu B.Cu) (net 3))
 (segment (start 63.5 50.8) (end 55.88 50.8) (width 0.25) (layer F.Cu) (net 3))
 (segment (start 55.88 53.34) (end 55.88 50.8) (width 0.25) (layer B.Cu) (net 3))
 (segment (start 55.88 53.34) (end 30.48 53.34) (width 0.25) (layer B.Cu) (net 3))
 (segment (start 17.78 53.34) (end 30.48 53.34) (width 0.25) (layer B.Cu) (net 3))
 (segment (start 30.48 53.34) (end 30.48 50.8) (width 0.25) (layer B.Cu) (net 3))
 (segment (start 17.78 53.34) (end 5.08 53.34) (width 0.25) (layer B.Cu) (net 3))
 (segment (start 5.08 53.34) (end 5.08 43.18) (width 0.25) (layer B.Cu) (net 3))
 (segment (start 17.78 50.8) (end 17.78 53.34) (width 0.25) (layer B.Cu) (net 3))
 (segment (start 10.16 30.48) (end 10.16 38.1) (width 0.25) (layer B.Cu) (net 3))
 (segment (start 10.16 38.1) (end 5.08 38.1) (width 0.25) (layer B.Cu) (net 3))
 (segment (start 5.08 38.1) (end 5.08 43.18) (width 0.25) (layer B.Cu) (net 3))
 (segment (start 38.1 43.9) (end 38.1 43.18) (width 0.25) (layer B.Cu) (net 3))
 (segment (start 38.1 43.18) (end 38.1 40.64) (width 0.25) (layer B.Cu) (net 3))
 (segment (start 9.44 30.48) (end 10.16 30.48) (width 0.25) (layer B.Cu) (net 3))
 (segment (start 27.94 48.26) (end 20.32 48.26) (width 0.25) (layer B.Cu) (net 4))
 (segment (start 20.32 48.26) (end 20.32 50.8) (width 0.25) (layer B.Cu) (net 4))
 (segment (start 10.16 15.24) (end 48.26 15.24) (width 0.25) (layer B.Cu) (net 5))
 (segment (start 48.26 15.24) (end 48.26 40.64) (width 0.25) (layer B.Cu) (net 5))
 (segment (start 45.72 40.64) (end 45.72 17.78) (width 0.25) (layer B.Cu) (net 7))
 (segment (start 45.72 17.78) (end 10.16 17.78) (width 0.25) (layer B.Cu) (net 7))
 (segment (start 10.16 20.32) (end 43.18 20.32) (width 0.25) (layer B.Cu) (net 9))
 (segment (start 43.18 20.32) (end 43.18 40.64) (width 0.25) (layer B.Cu) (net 9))
 (segment (start 53.34 48.26) (end 53.34 50.8) (width 0.25) (layer B.Cu) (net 2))
 (segment (start 53.34 50.8) (end 35.56 50.8) (width 0.25) (layer B.Cu) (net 2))
 (segment (start 35.56 50.8) (end 35.56 50.8) (width 0.25) (layer B.Cu) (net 2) (status 30))
 (segment (start 35.56 50.8) (end 35.56 50.8) (width 0.25) (layer B.Cu) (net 2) (status 10))
 (segment (start 35.56 50.8) (end 35.56 48.26) (width 0.25) (layer B.Cu) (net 2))
 (segment (start 40.64 40.64) (end 40.64 22.86) (width 0.25) (layer B.Cu) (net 10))
 (segment (start 40.64 22.86) (end 10.16 22.86) (width 0.25) (layer B.Cu) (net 10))
 (segment (start 40.64 48.26) (end 39.37 46.99) (width 0.25) (layer B.Cu) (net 11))
 (segment (start 8.89 24.13) (end 7.62 22.86) (width 0.25) (layer B.Cu) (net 11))
 (segment (start 39.37 24.13) (end 8.89 24.13) (width 0.25) (layer B.Cu) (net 11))
 (segment (start 39.37 41.91) (end 39.37 24.13) (width 0.25) (layer B.Cu) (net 11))
 (via (at 39.37 41.91) (size 0.6) (drill 0.4) (layers F.Cu B.Cu) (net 11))
 (segment (start 39.37 46.99) (end 39.37 41.91) (width 0.25) (layer F.Cu) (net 11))
 (via (at 39.37 46.99) (size 0.6) (drill 0.4) (layers F.Cu B.Cu) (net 11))
 (segment (start 7.62 20.32) (end 8.89 21.59) (width 0.25) (layer B.Cu) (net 13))
 (segment (start 41.91 46.99) (end 43.18 48.26) (width 0.25) (layer B.Cu) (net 13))
 (via (at 41.91 46.99) (size 0.6) (drill 0.4) (layers F.Cu B.Cu) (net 13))
 (segment (start 41.91 41.91) (end 41.91 46.99) (width 0.25) (layer F.Cu) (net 13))
 (via (at 41.91 41.91) (size 0.6) (drill 0.4) (layers F.Cu B.Cu) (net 13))
 (segment (start 41.91 21.59) (end 41.91 41.91) (width 0.25) (layer B.Cu) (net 13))
 (segment (start 8.89 21.59) (end 41.91 21.59) (width 0.25) (layer B.Cu) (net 13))
 (segment (start 7.62 25.4) (end 8.89 26.67) (width 0.25) (layer F.Cu) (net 14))
 (segment (start 33.02 26.67) (end 33.02 40.64) (width 0.25) (layer B.Cu) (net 14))
 (via (at 33.02 26.67) (size 0.6) (drill 0.4) (layers F.Cu B.Cu) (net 14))
 (segment (start 8.89 26.67) (end 33.02 26.67) (width 0.25) (layer F.Cu) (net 14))
 (segment (start 45.72 48.26) (end 44.45 46.99) (width 0.25) (layer B.Cu) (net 15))
 (segment (start 8.89 19.05) (end 7.62 17.78) (width 0.25) (layer B.Cu) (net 15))
 (segment (start 44.45 19.05) (end 8.89 19.05) (width 0.25) (layer B.Cu) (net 15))
 (segment (start 44.45 41.91) (end 44.45 19.05) (width 0.25) (layer B.Cu) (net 15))
 (via (at 44.45 41.91) (size 0.6) (drill 0.4) (layers F.Cu B.Cu) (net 15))
 (segment (start 44.45 46.99) (end 44.45 41.91) (width 0.25) (layer F.Cu) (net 15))
 (via (at 44.45 46.99) (size 0.6) (drill 0.4) (layers F.Cu B.Cu) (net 15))
 (segment (start 10.16 25.4) (end 30.48 25.4) (width 0.25) (layer B.Cu) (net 16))
 (segment (start 30.48 25.4) (end 30.48 40.64) (width 0.25) (layer B.Cu) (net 16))
 (segment (start 7.62 15.24) (end 8.89 16.51) (width 0.25) (layer B.Cu) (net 17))
 (segment (start 46.99 46.99) (end 48.26 48.26) (width 0.25) (layer B.Cu) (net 17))
 (via (at 46.99 46.99) (size 0.6) (drill 0.4) (layers F.Cu B.Cu) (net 17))
 (segment (start 46.99 41.91) (end 46.99 46.99) (width 0.25) (layer F.Cu) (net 17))
 (via (at 46.99 41.91) (size 0.6) (drill 0.4) (layers F.Cu B.Cu) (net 17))
 (segment (start 46.99 16.51) (end 46.99 41.91) (width 0.25) (layer B.Cu) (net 17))
 (segment (start 8.89 16.51) (end 46.99 16.51) (width 0.25) (layer B.Cu) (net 17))
 (segment (start 7.62 27.94) (end 8.89 26.67) (width 0.25) (layer B.Cu) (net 18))
 (segment (start 27.94 26.67) (end 27.94 40.64) (width 0.25) (layer B.Cu) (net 18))
 (segment (start 8.89 26.67) (end 27.94 26.67) (width 0.25) (layer B.Cu) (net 18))
 (segment (start 7.58 40.68) (end 12.66 40.68) (width 0.25) (layer B.Cu) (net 21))
 (segment (start 12.7 27.94) (end 12.66 27.98) (width 0.25) (layer B.Cu) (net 21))
 (segment (start 12.66 27.98) (end 12.66 40.68) (width 0.25) (layer B.Cu) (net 21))
 (segment (start 12.7 27.94) (end 10.16 27.94) (width 0.25) (layer B.Cu) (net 21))
 (segment (start 86.36 25.4) (end 86.36 20.32) (width 0.25) (layer B.Cu) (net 20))
 (segment (start 86.36 20.32) (end 88.9 20.32) (width 0.25) (layer B.Cu) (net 20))
 (segment (start 88.9 17.78) (end 88.9 20.32) (width 0.25) (layer B.Cu) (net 20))
 (segment (start 86.36 30.48) (end 86.36 40.64) (width 0.25) (layer B.Cu) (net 19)))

